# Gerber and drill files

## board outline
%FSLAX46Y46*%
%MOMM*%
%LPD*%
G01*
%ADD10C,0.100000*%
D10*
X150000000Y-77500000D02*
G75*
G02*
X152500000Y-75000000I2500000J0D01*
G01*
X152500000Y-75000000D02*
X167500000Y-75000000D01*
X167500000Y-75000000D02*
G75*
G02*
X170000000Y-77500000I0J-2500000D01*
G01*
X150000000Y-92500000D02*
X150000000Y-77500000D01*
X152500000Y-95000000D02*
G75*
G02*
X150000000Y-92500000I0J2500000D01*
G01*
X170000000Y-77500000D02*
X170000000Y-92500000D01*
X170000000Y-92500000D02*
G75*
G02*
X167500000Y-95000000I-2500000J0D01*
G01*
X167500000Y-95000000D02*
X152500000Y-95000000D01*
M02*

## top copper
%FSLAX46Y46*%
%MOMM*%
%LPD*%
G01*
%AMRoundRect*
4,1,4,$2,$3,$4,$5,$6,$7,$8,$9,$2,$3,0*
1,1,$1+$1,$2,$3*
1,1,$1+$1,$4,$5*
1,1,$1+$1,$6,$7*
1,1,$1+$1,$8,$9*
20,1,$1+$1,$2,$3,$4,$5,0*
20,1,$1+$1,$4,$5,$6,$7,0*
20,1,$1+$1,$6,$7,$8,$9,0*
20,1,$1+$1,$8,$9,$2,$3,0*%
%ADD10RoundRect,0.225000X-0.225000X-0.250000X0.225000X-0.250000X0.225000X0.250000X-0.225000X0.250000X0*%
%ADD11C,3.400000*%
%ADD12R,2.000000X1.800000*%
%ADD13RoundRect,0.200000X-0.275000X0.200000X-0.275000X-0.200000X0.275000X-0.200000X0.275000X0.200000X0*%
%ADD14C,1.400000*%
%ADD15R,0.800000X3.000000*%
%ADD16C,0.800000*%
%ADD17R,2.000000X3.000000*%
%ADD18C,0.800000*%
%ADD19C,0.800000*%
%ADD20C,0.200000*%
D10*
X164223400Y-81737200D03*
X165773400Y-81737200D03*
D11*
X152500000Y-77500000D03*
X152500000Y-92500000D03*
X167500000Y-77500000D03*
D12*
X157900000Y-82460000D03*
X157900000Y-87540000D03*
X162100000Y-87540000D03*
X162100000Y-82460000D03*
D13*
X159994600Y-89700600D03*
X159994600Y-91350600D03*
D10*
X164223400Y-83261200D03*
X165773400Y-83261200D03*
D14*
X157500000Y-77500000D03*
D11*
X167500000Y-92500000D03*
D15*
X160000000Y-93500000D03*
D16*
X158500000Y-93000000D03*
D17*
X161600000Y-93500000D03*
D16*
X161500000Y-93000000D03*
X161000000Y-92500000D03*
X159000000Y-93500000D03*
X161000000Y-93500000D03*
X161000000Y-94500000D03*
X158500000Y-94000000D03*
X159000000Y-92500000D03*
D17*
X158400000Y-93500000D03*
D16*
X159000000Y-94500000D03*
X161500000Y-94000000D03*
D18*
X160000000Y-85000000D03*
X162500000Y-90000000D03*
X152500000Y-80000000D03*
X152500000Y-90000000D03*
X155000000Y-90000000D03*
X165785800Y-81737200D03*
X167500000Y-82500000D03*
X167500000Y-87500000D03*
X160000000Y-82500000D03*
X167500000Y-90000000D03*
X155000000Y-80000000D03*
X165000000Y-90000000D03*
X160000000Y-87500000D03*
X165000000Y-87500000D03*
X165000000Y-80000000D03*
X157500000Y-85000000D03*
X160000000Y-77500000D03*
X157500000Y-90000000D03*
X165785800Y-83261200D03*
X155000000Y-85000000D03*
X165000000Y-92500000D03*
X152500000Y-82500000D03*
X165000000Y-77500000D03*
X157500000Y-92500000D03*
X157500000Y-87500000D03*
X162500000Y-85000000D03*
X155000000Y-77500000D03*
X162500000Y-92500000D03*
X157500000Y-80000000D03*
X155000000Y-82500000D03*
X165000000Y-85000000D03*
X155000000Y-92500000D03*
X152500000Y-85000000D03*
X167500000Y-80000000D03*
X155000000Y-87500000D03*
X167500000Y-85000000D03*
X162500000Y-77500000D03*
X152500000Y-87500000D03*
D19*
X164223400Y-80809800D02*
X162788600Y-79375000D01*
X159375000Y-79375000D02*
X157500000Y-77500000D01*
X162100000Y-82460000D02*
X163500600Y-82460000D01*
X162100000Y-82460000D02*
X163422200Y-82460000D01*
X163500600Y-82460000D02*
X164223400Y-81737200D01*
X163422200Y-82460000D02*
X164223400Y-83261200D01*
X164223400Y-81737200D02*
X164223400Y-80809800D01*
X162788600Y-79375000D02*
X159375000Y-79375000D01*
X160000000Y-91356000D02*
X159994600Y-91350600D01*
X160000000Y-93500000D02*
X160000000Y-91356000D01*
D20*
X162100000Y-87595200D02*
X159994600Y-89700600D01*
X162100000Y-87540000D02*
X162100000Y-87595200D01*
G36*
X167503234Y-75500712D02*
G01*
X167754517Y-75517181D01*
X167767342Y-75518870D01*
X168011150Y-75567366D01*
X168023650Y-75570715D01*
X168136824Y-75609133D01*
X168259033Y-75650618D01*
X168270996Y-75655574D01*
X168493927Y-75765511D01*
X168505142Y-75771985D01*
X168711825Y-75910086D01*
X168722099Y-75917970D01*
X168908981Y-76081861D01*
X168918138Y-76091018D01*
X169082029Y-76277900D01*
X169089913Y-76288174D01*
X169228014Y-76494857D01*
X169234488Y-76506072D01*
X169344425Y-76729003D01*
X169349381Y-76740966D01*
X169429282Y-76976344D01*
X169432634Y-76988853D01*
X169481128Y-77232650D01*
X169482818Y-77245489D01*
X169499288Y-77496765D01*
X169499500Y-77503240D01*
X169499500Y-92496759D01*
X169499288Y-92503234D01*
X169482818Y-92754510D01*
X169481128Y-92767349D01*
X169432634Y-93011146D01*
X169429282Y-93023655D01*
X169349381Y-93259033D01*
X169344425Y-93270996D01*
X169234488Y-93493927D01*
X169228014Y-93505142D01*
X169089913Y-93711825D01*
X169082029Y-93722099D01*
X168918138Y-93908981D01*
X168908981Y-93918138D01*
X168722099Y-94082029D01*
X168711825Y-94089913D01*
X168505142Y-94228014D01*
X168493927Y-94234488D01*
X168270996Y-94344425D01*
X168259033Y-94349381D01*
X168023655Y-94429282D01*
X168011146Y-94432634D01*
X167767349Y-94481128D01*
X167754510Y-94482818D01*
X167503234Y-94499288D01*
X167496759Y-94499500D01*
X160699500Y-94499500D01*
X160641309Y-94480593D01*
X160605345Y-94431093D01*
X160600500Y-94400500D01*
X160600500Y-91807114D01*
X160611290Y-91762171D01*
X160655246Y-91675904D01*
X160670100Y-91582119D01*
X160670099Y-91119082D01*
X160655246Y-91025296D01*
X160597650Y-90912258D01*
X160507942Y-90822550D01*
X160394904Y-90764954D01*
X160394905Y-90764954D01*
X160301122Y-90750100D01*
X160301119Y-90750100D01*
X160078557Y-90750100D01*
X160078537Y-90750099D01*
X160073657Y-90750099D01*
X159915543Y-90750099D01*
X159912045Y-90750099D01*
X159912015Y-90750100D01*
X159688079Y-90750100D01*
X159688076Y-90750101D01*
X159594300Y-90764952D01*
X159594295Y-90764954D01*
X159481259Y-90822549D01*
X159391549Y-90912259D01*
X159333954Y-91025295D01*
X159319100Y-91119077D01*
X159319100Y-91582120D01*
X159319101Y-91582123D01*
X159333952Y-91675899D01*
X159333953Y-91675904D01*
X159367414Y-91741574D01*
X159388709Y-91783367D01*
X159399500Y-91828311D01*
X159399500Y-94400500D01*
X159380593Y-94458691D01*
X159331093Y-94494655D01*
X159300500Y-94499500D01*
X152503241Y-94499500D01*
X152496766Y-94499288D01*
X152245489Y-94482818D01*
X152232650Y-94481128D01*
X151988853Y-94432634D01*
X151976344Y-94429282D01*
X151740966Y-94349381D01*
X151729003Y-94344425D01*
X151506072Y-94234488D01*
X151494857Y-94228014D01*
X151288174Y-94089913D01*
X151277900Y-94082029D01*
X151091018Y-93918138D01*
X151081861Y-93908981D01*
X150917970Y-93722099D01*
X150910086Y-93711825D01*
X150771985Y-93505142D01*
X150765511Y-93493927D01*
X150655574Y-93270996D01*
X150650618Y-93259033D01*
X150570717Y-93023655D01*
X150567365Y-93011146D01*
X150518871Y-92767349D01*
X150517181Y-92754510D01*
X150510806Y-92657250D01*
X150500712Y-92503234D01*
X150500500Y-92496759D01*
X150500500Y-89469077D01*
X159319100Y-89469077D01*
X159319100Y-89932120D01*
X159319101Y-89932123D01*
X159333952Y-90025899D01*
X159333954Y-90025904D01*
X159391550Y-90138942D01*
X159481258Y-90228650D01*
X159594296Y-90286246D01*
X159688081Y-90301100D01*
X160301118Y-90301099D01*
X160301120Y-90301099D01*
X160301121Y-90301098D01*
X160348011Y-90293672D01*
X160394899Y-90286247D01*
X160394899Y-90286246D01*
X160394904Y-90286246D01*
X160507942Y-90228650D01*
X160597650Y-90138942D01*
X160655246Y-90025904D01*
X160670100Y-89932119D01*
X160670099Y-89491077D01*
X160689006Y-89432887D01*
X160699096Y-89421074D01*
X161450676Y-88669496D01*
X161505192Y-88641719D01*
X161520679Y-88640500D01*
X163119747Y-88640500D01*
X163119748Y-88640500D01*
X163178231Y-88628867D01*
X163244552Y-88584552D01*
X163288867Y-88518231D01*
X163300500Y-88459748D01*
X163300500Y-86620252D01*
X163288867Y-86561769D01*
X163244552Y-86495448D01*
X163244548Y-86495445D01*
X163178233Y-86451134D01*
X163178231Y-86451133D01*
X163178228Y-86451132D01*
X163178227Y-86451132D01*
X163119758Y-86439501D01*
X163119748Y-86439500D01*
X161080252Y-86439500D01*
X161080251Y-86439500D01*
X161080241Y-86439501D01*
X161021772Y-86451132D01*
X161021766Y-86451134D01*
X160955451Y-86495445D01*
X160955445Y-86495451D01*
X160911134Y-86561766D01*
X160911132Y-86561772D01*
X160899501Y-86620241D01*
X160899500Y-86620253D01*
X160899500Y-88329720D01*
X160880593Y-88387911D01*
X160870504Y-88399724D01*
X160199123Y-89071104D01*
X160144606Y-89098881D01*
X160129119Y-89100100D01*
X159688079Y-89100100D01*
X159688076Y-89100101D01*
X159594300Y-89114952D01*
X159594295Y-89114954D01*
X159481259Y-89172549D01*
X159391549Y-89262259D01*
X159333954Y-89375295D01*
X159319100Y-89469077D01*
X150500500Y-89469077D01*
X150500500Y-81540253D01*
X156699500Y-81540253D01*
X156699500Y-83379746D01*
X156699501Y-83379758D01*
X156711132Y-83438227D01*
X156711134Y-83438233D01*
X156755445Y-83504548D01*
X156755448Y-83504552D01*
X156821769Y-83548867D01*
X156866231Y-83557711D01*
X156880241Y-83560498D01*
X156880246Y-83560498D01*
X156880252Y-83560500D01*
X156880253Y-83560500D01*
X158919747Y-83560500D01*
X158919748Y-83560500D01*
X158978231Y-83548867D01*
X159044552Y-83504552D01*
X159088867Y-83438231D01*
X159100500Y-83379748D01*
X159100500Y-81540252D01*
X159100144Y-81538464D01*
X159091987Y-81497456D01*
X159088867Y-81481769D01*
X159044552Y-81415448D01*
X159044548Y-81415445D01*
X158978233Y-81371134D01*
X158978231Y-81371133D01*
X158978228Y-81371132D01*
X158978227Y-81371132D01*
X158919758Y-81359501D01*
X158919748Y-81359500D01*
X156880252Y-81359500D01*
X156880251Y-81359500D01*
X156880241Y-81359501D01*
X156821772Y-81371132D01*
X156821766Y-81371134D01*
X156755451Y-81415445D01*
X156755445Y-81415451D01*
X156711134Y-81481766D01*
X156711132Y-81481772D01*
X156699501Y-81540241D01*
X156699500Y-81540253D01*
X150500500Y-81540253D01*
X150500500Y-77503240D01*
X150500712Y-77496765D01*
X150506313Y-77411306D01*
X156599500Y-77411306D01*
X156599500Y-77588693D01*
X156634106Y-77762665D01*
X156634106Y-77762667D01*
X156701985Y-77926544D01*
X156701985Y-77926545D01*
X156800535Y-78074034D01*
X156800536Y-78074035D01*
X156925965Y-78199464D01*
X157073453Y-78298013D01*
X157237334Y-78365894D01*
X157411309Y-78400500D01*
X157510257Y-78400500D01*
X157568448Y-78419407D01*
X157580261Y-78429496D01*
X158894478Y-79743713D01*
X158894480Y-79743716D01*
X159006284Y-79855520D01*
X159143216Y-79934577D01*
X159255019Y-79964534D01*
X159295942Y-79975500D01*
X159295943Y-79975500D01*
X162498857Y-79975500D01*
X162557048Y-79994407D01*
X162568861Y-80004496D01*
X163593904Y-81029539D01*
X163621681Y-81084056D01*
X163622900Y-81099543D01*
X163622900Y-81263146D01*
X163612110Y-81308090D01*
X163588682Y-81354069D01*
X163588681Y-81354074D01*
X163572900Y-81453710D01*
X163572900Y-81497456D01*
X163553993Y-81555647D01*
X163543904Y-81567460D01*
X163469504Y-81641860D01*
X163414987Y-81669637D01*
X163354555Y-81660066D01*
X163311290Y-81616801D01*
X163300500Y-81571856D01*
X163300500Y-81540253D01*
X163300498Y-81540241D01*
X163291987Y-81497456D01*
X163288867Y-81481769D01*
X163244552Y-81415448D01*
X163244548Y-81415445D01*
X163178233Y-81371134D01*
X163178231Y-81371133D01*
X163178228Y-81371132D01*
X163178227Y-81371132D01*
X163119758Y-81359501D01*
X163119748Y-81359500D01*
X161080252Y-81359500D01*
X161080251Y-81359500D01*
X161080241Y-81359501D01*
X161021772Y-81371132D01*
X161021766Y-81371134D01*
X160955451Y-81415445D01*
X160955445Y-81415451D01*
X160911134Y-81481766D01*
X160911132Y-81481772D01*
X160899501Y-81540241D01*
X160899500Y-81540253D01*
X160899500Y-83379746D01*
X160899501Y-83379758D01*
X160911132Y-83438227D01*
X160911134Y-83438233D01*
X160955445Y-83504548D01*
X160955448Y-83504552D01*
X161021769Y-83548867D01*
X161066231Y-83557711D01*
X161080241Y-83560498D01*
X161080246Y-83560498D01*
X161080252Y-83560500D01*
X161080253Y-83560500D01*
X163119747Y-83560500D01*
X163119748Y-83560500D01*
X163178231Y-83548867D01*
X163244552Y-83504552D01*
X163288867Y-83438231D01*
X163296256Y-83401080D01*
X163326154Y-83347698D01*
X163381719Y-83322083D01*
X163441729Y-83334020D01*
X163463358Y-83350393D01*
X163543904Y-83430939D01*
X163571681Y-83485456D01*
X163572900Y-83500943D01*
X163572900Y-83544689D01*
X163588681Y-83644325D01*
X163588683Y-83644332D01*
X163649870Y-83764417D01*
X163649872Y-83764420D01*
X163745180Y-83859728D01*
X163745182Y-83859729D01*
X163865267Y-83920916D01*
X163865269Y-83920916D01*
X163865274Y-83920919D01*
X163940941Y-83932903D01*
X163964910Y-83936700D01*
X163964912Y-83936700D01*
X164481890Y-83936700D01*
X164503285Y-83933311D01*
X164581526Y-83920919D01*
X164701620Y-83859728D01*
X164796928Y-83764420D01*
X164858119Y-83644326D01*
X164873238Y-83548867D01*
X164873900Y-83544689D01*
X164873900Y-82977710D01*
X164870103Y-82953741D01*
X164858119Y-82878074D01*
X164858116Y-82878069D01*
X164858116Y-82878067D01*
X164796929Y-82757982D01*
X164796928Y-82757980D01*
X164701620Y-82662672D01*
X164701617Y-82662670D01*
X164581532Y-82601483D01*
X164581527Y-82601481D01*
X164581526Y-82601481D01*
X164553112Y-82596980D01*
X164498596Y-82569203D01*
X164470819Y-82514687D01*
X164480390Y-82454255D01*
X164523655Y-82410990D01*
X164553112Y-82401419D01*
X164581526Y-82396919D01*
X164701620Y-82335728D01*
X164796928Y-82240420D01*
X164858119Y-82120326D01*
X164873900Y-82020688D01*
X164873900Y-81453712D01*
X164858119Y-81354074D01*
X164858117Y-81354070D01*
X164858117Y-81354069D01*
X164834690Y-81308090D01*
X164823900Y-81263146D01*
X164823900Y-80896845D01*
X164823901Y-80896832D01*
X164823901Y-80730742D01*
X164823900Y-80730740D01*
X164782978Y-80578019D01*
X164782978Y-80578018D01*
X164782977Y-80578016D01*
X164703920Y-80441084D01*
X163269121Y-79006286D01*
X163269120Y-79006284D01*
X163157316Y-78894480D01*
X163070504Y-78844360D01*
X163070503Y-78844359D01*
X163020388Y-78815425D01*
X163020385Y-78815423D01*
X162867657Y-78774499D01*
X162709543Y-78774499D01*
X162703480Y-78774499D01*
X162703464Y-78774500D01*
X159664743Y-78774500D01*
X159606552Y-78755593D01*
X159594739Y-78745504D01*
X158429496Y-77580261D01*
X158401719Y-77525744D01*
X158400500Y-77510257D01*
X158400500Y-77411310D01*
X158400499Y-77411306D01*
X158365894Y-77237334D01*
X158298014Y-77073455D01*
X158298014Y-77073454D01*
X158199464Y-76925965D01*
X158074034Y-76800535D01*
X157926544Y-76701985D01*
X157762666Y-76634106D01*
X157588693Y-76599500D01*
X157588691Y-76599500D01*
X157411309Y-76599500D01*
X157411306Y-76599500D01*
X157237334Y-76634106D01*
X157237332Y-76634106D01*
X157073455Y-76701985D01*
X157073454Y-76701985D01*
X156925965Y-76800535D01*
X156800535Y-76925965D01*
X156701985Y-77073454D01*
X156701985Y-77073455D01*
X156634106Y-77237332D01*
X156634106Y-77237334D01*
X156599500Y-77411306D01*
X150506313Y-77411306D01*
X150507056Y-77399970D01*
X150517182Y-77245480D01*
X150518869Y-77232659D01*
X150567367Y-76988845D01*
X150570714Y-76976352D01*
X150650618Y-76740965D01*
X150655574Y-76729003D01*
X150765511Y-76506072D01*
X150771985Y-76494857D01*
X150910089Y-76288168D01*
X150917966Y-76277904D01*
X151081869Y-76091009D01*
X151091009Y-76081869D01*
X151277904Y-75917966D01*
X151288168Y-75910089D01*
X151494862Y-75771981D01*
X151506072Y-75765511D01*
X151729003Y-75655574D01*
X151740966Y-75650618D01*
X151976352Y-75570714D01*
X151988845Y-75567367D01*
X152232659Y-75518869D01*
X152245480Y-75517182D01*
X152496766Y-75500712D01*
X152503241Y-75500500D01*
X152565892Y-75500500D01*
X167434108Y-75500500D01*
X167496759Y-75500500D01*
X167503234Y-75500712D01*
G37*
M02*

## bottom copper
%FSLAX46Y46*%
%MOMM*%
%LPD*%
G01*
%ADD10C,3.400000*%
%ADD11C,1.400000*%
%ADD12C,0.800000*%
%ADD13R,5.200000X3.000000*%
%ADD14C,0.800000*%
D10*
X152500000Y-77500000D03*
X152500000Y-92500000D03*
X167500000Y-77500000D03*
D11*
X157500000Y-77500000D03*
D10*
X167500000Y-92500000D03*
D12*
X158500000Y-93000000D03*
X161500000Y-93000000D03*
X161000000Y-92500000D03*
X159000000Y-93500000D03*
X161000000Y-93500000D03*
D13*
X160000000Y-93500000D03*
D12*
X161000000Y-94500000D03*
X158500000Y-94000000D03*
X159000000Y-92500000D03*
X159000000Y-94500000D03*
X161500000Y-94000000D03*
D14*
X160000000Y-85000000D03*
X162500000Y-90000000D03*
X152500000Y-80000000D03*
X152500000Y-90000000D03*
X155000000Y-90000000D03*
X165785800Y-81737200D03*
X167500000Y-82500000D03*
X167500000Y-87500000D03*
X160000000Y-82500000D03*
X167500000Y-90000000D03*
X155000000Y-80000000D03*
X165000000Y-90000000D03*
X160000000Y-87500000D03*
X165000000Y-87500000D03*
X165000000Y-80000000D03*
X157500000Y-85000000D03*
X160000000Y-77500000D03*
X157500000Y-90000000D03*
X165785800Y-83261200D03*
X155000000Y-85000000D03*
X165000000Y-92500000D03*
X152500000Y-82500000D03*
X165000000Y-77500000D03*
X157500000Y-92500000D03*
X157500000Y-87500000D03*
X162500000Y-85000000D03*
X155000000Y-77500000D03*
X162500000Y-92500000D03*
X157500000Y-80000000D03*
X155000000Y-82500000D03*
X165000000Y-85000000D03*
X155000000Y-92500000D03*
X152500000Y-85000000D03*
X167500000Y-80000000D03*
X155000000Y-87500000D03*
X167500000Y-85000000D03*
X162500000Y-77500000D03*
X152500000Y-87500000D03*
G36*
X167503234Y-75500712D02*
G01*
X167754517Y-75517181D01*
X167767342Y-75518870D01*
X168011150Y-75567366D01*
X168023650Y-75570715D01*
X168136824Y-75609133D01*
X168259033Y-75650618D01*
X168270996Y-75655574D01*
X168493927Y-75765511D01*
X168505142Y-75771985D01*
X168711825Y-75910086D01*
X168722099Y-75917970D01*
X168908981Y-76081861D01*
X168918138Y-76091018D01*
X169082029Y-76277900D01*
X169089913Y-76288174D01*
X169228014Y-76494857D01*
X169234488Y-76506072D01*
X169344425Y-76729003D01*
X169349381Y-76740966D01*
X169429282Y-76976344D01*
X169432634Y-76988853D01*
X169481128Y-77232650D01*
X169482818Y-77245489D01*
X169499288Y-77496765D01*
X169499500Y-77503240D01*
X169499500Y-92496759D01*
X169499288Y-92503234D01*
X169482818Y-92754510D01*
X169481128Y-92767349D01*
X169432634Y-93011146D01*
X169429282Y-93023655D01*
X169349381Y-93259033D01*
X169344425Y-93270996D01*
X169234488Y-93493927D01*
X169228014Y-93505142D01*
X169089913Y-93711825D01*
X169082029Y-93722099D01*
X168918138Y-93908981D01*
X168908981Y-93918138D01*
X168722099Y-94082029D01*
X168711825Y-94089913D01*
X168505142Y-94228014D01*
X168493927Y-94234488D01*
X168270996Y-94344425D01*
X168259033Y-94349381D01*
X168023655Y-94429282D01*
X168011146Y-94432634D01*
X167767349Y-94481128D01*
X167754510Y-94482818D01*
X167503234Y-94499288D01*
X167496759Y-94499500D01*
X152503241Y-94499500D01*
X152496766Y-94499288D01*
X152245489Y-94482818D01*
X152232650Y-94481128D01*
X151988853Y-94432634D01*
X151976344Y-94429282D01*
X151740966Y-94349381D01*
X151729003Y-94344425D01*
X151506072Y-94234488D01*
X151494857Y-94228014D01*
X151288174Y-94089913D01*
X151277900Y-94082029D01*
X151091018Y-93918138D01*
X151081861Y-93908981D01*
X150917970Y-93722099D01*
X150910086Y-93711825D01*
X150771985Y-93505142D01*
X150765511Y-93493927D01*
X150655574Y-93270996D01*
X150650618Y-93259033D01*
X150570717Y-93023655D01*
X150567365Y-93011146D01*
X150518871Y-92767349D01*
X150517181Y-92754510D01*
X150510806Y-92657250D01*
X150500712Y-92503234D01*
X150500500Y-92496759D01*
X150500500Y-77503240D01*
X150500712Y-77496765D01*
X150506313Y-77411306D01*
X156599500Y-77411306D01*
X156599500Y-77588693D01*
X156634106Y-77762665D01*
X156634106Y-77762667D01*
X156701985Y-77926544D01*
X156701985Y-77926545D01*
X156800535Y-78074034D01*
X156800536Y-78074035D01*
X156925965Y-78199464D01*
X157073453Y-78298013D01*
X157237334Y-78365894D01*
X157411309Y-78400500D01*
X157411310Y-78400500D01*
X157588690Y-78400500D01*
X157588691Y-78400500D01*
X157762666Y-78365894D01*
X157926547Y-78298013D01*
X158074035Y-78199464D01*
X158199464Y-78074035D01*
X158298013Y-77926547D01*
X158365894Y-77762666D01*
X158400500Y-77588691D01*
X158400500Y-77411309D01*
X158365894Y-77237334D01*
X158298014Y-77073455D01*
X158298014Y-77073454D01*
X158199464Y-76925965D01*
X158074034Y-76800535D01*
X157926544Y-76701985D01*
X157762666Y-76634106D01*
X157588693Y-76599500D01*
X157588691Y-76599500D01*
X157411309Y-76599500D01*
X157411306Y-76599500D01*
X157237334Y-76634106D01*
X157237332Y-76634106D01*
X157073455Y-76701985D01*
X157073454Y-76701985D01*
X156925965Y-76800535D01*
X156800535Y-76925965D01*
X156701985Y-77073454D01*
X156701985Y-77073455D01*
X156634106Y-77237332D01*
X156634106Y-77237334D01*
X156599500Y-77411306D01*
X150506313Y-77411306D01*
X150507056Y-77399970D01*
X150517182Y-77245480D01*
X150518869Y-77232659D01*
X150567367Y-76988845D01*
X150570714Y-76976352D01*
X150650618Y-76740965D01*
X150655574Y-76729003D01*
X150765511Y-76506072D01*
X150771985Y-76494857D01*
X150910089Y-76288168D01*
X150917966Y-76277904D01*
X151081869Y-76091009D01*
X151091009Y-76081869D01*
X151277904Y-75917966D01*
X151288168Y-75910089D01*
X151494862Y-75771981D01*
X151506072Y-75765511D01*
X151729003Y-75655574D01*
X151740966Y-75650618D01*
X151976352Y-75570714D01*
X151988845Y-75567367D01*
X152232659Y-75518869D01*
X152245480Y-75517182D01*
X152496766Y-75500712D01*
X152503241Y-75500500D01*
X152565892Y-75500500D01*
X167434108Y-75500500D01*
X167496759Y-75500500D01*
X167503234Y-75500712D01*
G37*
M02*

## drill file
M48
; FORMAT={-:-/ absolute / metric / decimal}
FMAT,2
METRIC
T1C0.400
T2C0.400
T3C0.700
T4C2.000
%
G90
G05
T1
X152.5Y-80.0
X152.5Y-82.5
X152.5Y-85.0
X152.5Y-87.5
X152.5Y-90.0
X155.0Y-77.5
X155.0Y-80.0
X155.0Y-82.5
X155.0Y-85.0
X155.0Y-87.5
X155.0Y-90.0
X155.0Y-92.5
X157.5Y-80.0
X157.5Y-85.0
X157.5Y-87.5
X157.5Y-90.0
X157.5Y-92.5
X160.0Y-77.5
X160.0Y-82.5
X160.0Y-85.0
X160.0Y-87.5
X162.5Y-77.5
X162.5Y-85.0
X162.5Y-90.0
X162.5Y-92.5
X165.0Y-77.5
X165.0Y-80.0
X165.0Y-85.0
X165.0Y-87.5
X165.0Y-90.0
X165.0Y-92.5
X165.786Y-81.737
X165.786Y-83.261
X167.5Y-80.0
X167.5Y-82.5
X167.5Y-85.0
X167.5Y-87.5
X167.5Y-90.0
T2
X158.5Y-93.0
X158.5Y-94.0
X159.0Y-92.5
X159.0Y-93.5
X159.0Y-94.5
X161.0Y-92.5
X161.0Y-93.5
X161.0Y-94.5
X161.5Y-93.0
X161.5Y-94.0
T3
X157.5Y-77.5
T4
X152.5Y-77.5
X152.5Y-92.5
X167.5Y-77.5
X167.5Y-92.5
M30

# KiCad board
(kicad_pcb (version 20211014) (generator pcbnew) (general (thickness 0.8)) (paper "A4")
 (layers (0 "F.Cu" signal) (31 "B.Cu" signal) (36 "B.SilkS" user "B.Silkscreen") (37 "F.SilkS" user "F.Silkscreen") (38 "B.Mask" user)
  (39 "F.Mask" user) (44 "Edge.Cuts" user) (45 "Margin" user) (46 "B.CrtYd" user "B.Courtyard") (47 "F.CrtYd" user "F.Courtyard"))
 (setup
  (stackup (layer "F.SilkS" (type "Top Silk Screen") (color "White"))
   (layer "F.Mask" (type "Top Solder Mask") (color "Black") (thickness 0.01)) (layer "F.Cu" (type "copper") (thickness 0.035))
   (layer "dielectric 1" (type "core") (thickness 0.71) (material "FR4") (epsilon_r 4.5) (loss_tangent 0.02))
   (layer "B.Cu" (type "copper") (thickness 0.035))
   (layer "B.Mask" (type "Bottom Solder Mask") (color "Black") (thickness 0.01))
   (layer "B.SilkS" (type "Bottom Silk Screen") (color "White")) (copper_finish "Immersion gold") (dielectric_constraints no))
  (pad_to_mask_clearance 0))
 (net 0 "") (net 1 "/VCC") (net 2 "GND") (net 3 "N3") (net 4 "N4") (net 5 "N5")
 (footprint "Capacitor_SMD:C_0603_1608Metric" (layer "F.Cu") (at 164.9984 81.7372)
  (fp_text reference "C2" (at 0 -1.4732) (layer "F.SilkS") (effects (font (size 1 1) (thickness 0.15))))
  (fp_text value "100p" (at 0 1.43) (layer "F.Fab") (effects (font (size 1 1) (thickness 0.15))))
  (pad "1" smd roundrect (at -0.775 0) (size 0.9 0.95) (layers "F.Cu" "F.Paste" "F.Mask") (roundrect_rratio 0.25) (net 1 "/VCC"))
  (pad "2" smd roundrect (at 0.775 0) (size 0.9 0.95) (layers "F.Cu" "F.Paste" "F.Mask") (roundrect_rratio 0.25) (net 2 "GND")))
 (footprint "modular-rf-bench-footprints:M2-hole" (layer "F.Cu") (at 152.5 77.5)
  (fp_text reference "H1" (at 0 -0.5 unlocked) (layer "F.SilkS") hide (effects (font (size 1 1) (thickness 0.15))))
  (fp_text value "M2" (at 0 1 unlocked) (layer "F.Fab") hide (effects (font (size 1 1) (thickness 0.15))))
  (pad "1" thru_hole circle (at 0 0) (size 3.4 3.4) (drill 2) (layers *.Cu *.Mask) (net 2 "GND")))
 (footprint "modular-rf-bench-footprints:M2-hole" (layer "F.Cu") (at 152.5 92.5)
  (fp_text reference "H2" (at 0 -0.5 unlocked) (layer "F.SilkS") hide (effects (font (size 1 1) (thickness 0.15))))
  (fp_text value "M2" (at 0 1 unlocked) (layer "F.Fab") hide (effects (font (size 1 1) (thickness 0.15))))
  (pad "1" thru_hole circle (at 0 0) (size 3.4 3.4) (drill 2) (layers *.Cu *.Mask) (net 2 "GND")))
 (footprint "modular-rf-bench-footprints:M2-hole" (layer "F.Cu") (at 167.5 77.5)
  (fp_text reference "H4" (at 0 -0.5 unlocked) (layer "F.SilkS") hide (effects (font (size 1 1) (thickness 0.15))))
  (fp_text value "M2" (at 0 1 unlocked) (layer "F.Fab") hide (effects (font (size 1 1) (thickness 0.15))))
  (pad "1" thru_hole circle (at 0 0) (size 3.4 3.4) (drill 2) (layers *.Cu *.Mask) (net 2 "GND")))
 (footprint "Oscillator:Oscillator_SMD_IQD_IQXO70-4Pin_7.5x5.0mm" (layer "F.Cu") (at 160 85 -90)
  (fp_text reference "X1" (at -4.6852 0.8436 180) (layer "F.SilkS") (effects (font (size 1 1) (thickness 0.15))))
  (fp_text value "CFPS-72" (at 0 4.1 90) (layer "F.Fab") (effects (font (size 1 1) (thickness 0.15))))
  (pad "1" smd rect (at -2.54 2.1 270) (size 1.8 2) (layers "F.Cu" "F.Paste" "F.Mask") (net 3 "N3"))
  (pad "2" smd rect (at 2.54 2.1 270) (size 1.8 2) (layers "F.Cu" "F.Paste" "F.Mask") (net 2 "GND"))
  (pad "3" smd rect (at 2.54 -2.1 270) (size 1.8 2) (layers "F.Cu" "F.Paste" "F.Mask") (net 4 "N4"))
  (pad "4" smd rect (at -2.54 -2.1 270) (size 1.8 2) (layers "F.Cu" "F.Paste" "F.Mask") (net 1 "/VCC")))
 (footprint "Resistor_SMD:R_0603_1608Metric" (layer "F.Cu") (at 159.9946 90.5256 -90)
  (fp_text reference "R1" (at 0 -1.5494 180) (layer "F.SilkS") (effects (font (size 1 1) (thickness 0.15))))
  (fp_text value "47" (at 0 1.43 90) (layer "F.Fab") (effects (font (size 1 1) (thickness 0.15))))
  (pad "1" smd roundrect (at -0.825 0 270) (size 0.8 0.95) (layers "F.Cu" "F.Paste" "F.Mask") (roundrect_rratio 0.25) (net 4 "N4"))
  (pad "2" smd roundrect (at 0.825 0 270) (size 0.8 0.95) (layers "F.Cu" "F.Paste" "F.Mask") (roundrect_rratio 0.25) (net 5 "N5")))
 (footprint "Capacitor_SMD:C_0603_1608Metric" (layer "F.Cu") (at 164.9984 83.2612)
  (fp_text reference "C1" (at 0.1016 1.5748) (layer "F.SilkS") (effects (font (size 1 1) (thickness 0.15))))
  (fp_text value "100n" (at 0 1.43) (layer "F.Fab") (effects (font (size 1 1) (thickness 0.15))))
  (pad "1" smd roundrect (at -0.775 0) (size 0.9 0.95) (layers "F.Cu" "F.Paste" "F.Mask") (roundrect_rratio 0.25) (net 1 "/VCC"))
  (pad "2" smd roundrect (at 0.775 0) (size 0.9 0.95) (layers "F.Cu" "F.Paste" "F.Mask") (roundrect_rratio 0.25) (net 2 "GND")))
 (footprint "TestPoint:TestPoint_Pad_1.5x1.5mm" (layer "F.Cu") (at 157.5 77.5)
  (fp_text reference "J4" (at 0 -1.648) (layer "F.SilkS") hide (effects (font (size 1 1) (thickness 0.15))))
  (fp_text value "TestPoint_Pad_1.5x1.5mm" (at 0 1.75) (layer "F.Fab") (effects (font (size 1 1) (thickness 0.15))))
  (pad "1" thru_hole circle (at 0 0) (size 1.4 1.4) (drill 0.7) (layers *.Cu *.Mask) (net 1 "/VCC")))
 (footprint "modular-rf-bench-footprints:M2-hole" (layer "F.Cu") (at 167.5 92.5)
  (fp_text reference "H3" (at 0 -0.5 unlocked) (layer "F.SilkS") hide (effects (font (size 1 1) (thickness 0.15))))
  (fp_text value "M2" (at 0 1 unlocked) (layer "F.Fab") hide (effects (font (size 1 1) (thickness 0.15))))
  (pad "1" thru_hole circle (at 0 0) (size 3.4 3.4) (drill 2) (layers *.Cu *.Mask) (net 2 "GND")))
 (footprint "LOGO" (layer "F.Cu") (at 164.592 89.916)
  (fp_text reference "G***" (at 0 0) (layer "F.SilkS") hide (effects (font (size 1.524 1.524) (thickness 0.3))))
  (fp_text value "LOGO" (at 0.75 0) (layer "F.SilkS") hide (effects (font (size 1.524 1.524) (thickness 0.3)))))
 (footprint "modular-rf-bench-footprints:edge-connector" (layer "F.Cu") (at 160 95 -90)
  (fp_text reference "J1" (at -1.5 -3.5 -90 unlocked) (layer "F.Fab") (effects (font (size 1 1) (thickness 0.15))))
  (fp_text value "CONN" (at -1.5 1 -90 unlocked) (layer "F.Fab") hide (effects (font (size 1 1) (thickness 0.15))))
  (pad "1" smd rect (at -1.5 0 270) (size 3 0.8) (layers "F.Cu") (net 5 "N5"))
  (pad "2" thru_hole circle (at -2 1.5 270) (size 0.8 0.8) (drill 0.4) (layers *.Cu) (remove_unused_layers) (keep_end_layers) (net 2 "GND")
   (zone_connect 2))
  (pad "2" smd rect (at -1.5 -1.6 270) (size 3 2) (layers "F.Cu") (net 2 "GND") (zone_connect 2))
  (pad "2" thru_hole circle (at -2 -1.5 270) (size 0.8 0.8) (drill 0.4) (layers *.Cu) (remove_unused_layers) (keep_end_layers) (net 2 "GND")
   (zone_connect 2))
  (pad "2" thru_hole circle (at -2.5 -1 270) (size 0.8 0.8) (drill 0.4) (layers *.Cu) (remove_unused_layers) (keep_end_layers) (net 2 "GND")
   (zone_connect 2))
  (pad "2" thru_hole circle (at -1.5 1 270) (size 0.8 0.8) (drill 0.4) (layers *.Cu) (remove_unused_layers) (keep_end_layers) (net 2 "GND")
   (zone_connect 2))
  (pad "2" thru_hole circle (at -1.5 -1 270) (size 0.8 0.8) (drill 0.4) (layers *.Cu) (remove_unused_layers) (keep_end_layers) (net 2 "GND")
   (zone_connect 2))
  (pad "2" smd rect (at -1.5 0 270) (size 3 5.2) (layers "B.Cu") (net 2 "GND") (zone_connect 2))
  (pad "2" thru_hole circle (at -0.5 -1 270) (size 0.8 0.8) (drill 0.4) (layers *.Cu) (remove_unused_layers) (keep_end_layers) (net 2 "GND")
   (zone_connect 2))
  (pad "2" thru_hole circle (at -1 1.5 270) (size 0.8 0.8) (drill 0.4) (layers *.Cu) (remove_unused_layers) (keep_end_layers) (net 2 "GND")
   (zone_connect 2))
  (pad "2" thru_hole circle (at -2.5 1 270) (size 0.8 0.8) (drill 0.4) (layers *.Cu) (remove_unused_layers) (keep_end_layers) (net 2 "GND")
   (zone_connect 2))
  (pad "2" smd rect (at -1.5 1.6 270) (size 3 2) (layers "F.Cu") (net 2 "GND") (zone_connect 2))
  (pad "2" thru_hole circle (at -0.5 1 270) (size 0.8 0.8) (drill 0.4) (layers *.Cu) (remove_unused_layers) (keep_end_layers) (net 2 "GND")
   (zone_connect 2))
  (pad "2" thru_hole circle (at -1 -1.5 270) (size 0.8 0.8) (drill 0.4) (layers *.Cu) (remove_unused_layers) (keep_end_layers) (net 2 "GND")
   (zone_connect 2)))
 (gr_arc (start 150 77.5) (mid 150.732233 75.732233) (end 152.5 75) (layer "Edge.Cuts") (width 0.1))
 (gr_line (start 152.5 75) (end 167.5 75) (layer "Edge.Cuts") (width 0.1))
 (gr_arc (start 167.5 75) (mid 169.267767 75.732233) (end 170 77.5) (layer "Edge.Cuts") (width 0.1))
 (gr_line (start 150 92.5) (end 150 77.5) (layer "Edge.Cuts") (width 0.1))
 (gr_arc (start 152.5 95) (mid 150.732233 94.267767) (end 150 92.5) (layer "Edge.Cuts") (width 0.1))
 (gr_line (start 170 77.5) (end 170 92.5) (layer "Edge.Cuts") (width 0.1))
 (gr_arc (start 170 92.5) (mid 169.267767 94.267767) (end 167.5 95) (layer "Edge.Cuts") (width 0.1))
 (gr_line (start 167.5 95) (end 152.5 95) (layer "Edge.Cuts") (width 0.1))
 (via (at 160 85) (size 0.8) (drill 0.4) (layers "F.Cu" "B.Cu") (free) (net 2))
 (via (at 162.5 90) (size 0.8) (drill 0.4) (layers "F.Cu" "B.Cu") (free) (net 2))
 (via (at 152.5 80) (size 0.8) (drill 0.4) (layers "F.Cu" "B.Cu") (free) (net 2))
 (via (at 152.5 90) (size 0.8) (drill 0.4) (layers "F.Cu" "B.Cu") (free) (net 2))
 (via (at 155 90) (size 0.8) (drill 0.4) (layers "F.Cu" "B.Cu") (free) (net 2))
 (via (at 165.7858 81.7372) (size 0.8) (drill 0.4) (layers "F.Cu" "B.Cu") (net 2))
 (via (at 167.5 82.5) (size 0.8) (drill 0.4) (layers "F.Cu" "B.Cu") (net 2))
 (via (at 167.5 87.5) (size 0.8) (drill 0.4) (layers "F.Cu" "B.Cu") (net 2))
 (via (at 160 82.5) (size 0.8) (drill 0.4) (layers "F.Cu" "B.Cu") (free) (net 2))
 (via (at 167.5 90) (size 0.8) (drill 0.4) (layers "F.Cu" "B.Cu") (free) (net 2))
 (via (at 155 80) (size 0.8) (drill 0.4) (layers "F.Cu" "B.Cu") (free) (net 2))
 (via (at 165 90) (size 0.8) (drill 0.4) (layers "F.Cu" "B.Cu") (free) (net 2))
 (via (at 160 87.5) (size 0.8) (drill 0.4) (layers "F.Cu" "B.Cu") (free) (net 2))
 (via (at 165 87.5) (size 0.8) (drill 0.4) (layers "F.Cu" "B.Cu") (free) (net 2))
 (via (at 165 80) (size 0.8) (drill 0.4) (layers "F.Cu" "B.Cu") (free) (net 2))
 (via (at 157.5 85) (size 0.8) (drill 0.4) (layers "F.Cu" "B.Cu") (free) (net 2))
 (via (at 160 77.5) (size 0.8) (drill 0.4) (layers "F.Cu" "B.Cu") (free) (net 2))
 (via (at 157.5 90) (size 0.8) (drill 0.4) (layers "F.Cu" "B.Cu") (free) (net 2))
 (via (at 165.7858 83.2612) (size 0.8) (drill 0.4) (layers "F.Cu" "B.Cu") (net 2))
 (via (at 155 85) (size 0.8) (drill 0.4) (layers "F.Cu" "B.Cu") (free) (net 2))
 (via (at 165 92.5) (size 0.8) (drill 0.4) (layers "F.Cu" "B.Cu") (free) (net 2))
 (via (at 152.5 82.5) (size 0.8) (drill 0.4) (layers "F.Cu" "B.Cu") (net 2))
 (via (at 165 77.5) (size 0.8) (drill 0.4) (layers "F.Cu" "B.Cu") (free) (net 2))
 (via (at 157.5 92.5) (size 0.8) (drill 0.4) (layers "F.Cu" "B.Cu") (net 2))
 (via (at 157.5 87.5) (size 0.8) (drill 0.4) (layers "F.Cu" "B.Cu") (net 2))
 (via (at 162.5 85) (size 0.8) (drill 0.4) (layers "F.Cu" "B.Cu") (free) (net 2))
 (via (at 155 77.5) (size 0.8) (drill 0.4) (layers "F.Cu" "B.Cu") (free) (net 2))
 (via (at 162.5 92.5) (size 0.8) (drill 0.4) (layers "F.Cu" "B.Cu") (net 2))
 (via (at 157.5 80) (size 0.8) (drill 0.4) (layers "F.Cu" "B.Cu") (free) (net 2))
 (via (at 155 82.5) (size 0.8) (drill 0.4) (layers "F.Cu" "B.Cu") (free) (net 2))
 (via (at 165 85) (size 0.8) (drill 0.4) (layers "F.Cu" "B.Cu") (free) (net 2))
 (via (at 155 92.5) (size 0.8) (drill 0.4) (layers "F.Cu" "B.Cu") (free) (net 2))
 (via (at 152.5 85) (size 0.8) (drill 0.4) (layers "F.Cu" "B.Cu") (free) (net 2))
 (via (at 167.5 80) (size 0.8) (drill 0.4) (layers "F.Cu" "B.Cu") (free) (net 2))
 (via (at 155 87.5) (size 0.8) (drill 0.4) (layers "F.Cu" "B.Cu") (free) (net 2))
 (via (at 167.5 85) (size 0.8) (drill 0.4) (layers "F.Cu" "B.Cu") (free) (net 2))
 (via (at 162.5 77.5) (size 0.8) (drill 0.4) (layers "F.Cu" "B.Cu") (free) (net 2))
 (via (at 152.5 87.5) (size 0.8) (drill 0.4) (layers "F.Cu" "B.Cu") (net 2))
 (segment (start 164.2234 80.8098) (end 162.7886 79.375) (width 0.8) (layer "F.Cu") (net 1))
 (segment (start 159.375 79.375) (end 157.5 77.5) (width 0.8) (layer "F.Cu") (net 1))
 (segment (start 162.1 82.46) (end 163.5006 82.46) (width 0.8) (layer "F.Cu") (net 1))
 (segment (start 162.1 82.46) (end 163.4222 82.46) (width 0.8) (layer "F.Cu") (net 1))
 (segment (start 163.5006 82.46) (end 164.2234 81.7372) (width 0.8) (layer "F.Cu") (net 1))
 (segment (start 163.4222 82.46) (end 164.2234 83.2612) (width 0.8) (layer "F.Cu") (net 1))
 (segment (start 164.2234 81.7372) (end 164.2234 80.8098) (width 0.8) (layer "F.Cu") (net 1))
 (segment (start 162.7886 79.375) (end 159.375 79.375) (width 0.8) (layer "F.Cu") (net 1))
 (segment (start 160 91.356) (end 159.9946 91.3506) (width 0.8) (layer "F.Cu") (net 5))
 (segment (start 160 93.5) (end 160 91.356) (width 0.8) (layer "F.Cu") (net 5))
 (segment (start 162.1 87.5952) (end 159.9946 89.7006) (width 0.2) (layer "F.Cu") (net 4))
 (segment (start 162.1 87.54) (end 162.1 87.5952) (width 0.2) (layer "F.Cu") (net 4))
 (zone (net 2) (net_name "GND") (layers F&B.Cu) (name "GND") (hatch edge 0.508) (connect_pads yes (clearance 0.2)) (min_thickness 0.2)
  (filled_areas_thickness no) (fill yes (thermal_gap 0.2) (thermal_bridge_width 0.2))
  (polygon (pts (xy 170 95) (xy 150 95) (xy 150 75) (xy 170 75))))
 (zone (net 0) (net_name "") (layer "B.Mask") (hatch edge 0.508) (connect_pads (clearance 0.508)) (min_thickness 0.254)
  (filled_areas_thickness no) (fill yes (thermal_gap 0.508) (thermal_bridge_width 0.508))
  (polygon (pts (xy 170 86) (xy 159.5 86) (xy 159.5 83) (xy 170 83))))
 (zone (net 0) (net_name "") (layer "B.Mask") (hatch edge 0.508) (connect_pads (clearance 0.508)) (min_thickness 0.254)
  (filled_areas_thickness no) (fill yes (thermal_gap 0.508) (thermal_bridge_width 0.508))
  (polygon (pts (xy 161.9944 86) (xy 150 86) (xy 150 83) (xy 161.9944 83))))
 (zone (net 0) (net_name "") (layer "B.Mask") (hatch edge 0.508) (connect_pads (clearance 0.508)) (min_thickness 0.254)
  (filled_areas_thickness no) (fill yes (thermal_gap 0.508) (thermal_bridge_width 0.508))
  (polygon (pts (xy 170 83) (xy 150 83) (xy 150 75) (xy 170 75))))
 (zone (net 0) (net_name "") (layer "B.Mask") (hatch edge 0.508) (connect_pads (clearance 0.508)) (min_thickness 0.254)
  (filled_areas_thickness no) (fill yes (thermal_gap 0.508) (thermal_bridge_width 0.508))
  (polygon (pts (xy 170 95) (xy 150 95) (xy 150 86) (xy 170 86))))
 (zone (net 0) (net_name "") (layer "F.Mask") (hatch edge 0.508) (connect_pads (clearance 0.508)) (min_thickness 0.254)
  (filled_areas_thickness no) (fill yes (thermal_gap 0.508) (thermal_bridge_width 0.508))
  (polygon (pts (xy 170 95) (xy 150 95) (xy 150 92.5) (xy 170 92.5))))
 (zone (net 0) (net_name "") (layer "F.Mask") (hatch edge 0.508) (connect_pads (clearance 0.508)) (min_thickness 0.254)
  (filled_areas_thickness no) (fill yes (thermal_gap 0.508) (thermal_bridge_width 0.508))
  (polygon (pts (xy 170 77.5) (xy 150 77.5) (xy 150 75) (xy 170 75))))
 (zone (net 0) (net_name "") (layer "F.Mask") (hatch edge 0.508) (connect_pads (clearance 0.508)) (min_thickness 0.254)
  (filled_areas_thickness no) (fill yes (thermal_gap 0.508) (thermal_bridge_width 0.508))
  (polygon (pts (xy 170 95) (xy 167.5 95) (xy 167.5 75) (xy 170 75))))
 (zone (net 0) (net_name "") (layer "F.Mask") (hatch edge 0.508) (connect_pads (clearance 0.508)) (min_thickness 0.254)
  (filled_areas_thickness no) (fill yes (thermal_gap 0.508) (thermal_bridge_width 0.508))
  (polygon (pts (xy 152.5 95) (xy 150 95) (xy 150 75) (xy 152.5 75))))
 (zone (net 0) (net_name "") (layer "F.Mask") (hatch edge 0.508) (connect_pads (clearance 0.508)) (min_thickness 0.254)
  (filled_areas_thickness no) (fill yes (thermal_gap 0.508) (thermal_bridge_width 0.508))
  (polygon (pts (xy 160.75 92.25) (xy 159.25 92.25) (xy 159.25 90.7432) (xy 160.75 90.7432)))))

